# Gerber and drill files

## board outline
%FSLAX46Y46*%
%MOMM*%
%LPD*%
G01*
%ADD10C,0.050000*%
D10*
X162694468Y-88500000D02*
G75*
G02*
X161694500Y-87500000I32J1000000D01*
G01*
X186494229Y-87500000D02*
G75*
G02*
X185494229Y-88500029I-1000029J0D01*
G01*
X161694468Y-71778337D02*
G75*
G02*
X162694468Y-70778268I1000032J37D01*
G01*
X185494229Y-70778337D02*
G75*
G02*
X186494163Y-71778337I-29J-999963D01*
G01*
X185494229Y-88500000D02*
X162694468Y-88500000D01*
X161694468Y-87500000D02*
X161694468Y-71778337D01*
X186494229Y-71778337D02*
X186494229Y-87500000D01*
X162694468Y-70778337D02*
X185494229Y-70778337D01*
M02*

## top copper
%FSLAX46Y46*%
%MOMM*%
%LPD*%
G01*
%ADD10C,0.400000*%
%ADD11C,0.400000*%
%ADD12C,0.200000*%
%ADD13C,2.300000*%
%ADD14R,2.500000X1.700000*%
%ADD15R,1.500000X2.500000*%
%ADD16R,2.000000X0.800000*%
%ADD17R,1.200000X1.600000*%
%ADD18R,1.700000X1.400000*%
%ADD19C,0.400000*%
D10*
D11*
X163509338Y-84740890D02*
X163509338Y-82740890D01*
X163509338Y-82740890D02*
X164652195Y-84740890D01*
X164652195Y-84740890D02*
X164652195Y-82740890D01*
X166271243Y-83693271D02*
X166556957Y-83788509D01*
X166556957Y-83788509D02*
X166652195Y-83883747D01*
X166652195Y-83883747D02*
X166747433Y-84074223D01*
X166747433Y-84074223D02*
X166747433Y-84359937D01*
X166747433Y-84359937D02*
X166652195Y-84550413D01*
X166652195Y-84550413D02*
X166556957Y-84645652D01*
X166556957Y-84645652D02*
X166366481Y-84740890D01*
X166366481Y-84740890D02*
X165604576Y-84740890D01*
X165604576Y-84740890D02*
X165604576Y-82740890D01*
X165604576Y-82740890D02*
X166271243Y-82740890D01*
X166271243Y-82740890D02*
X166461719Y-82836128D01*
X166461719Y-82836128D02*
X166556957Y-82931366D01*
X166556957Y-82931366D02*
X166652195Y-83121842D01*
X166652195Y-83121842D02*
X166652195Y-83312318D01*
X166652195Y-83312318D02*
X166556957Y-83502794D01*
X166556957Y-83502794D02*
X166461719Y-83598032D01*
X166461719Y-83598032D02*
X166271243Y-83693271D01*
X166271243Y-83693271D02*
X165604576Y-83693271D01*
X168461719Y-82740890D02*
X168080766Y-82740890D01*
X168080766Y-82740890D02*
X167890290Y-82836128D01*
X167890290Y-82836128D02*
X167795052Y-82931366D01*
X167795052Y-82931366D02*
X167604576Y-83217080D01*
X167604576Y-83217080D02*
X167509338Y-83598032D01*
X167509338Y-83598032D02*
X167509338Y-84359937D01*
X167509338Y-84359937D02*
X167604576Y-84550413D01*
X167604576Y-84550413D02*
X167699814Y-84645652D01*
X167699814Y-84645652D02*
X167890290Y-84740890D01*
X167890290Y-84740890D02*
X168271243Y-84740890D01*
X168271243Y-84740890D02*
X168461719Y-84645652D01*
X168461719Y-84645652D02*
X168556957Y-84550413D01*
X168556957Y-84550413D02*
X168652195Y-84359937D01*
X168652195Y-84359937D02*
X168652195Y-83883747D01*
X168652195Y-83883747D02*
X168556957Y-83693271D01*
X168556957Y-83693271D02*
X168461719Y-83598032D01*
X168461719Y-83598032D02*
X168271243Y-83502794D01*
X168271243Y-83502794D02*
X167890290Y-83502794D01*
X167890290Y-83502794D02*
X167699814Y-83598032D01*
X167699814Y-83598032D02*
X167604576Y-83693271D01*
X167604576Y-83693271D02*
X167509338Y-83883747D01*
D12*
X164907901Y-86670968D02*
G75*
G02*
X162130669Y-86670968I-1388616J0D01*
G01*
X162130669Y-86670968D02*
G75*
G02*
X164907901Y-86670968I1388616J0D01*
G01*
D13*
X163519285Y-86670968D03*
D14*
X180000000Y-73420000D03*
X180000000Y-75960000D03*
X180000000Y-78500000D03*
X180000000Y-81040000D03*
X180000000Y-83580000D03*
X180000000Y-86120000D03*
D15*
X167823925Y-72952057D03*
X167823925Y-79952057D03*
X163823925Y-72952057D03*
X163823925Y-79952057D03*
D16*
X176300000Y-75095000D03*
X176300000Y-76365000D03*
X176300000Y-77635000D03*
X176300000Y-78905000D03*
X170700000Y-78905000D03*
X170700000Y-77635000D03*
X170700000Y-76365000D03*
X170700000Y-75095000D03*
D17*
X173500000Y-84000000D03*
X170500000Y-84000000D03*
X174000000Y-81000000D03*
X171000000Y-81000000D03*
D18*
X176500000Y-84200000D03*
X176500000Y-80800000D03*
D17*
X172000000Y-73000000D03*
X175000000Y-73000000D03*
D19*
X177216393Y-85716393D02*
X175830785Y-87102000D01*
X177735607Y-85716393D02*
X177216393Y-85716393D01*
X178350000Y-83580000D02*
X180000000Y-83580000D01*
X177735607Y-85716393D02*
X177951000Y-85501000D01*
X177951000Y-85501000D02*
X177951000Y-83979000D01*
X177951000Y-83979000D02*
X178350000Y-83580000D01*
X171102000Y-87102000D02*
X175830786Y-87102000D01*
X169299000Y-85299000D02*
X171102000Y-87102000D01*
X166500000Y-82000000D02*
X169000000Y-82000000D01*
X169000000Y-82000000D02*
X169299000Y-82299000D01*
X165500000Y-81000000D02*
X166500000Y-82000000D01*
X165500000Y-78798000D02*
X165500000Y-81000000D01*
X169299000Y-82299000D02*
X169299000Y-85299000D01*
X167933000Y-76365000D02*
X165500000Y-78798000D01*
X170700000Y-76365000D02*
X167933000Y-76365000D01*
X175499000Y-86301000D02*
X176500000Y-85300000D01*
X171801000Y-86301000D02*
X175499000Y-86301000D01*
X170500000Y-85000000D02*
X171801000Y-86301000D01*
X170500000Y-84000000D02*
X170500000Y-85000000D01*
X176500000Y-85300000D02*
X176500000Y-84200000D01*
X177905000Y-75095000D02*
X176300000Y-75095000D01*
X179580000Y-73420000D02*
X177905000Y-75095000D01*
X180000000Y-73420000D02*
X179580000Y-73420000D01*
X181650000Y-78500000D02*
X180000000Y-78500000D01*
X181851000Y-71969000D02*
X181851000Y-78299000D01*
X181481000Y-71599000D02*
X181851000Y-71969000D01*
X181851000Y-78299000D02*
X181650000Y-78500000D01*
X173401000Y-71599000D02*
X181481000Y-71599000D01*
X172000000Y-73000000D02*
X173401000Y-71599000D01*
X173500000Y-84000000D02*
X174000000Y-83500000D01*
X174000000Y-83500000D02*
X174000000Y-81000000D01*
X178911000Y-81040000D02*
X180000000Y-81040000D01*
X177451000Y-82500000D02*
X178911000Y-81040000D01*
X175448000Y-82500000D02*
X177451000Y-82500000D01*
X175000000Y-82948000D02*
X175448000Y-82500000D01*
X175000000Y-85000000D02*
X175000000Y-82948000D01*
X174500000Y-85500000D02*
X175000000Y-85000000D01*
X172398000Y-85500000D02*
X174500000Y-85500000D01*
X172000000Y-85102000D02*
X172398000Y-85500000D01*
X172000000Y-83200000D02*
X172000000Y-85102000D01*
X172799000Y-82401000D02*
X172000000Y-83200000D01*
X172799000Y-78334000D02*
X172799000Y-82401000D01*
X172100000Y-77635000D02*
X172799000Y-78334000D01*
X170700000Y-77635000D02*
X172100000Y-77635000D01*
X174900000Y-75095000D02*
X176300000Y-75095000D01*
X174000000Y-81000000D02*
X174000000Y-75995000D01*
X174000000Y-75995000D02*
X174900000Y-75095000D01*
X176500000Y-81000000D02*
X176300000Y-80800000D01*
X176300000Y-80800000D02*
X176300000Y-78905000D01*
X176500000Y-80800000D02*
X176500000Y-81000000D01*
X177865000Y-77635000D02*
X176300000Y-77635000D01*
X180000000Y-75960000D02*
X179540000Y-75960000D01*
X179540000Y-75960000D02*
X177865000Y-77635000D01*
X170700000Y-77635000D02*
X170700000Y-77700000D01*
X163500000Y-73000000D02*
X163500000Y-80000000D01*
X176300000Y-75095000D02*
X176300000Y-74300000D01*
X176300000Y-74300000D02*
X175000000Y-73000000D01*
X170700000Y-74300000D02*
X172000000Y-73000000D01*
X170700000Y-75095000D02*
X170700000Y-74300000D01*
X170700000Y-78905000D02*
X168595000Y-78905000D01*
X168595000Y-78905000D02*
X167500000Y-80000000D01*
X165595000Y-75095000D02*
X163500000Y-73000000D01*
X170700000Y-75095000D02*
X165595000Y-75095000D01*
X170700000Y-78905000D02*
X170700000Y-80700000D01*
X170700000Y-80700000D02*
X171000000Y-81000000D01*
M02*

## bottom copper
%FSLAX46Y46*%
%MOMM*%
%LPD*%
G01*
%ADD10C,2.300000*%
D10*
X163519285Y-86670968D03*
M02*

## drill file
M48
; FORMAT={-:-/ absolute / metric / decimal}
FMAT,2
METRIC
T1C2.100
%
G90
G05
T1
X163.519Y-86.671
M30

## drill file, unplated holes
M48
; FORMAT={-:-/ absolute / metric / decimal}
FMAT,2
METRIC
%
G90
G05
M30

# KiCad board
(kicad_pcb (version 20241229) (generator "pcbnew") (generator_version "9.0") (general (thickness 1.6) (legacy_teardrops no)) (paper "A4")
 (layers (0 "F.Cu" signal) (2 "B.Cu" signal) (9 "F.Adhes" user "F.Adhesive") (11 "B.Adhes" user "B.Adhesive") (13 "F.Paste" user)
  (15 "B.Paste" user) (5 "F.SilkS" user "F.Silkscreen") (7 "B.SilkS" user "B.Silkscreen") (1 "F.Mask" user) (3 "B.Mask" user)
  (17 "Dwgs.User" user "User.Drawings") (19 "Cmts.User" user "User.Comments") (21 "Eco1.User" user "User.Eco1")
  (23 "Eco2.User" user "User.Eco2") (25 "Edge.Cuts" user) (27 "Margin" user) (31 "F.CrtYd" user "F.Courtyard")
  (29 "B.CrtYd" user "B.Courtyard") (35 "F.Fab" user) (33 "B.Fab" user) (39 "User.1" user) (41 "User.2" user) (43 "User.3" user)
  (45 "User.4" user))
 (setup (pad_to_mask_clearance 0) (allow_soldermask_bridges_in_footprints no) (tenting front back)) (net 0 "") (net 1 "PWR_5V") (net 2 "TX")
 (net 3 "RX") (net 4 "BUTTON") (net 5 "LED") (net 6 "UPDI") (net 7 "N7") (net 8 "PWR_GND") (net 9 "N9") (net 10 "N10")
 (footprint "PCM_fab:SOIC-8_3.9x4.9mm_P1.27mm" (layer "F.Cu") (at 173.5 77)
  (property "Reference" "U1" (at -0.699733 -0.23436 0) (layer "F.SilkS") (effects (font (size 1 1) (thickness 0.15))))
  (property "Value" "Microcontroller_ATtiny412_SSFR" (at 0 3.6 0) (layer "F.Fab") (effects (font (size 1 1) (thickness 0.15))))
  (pad "1" smd rect (at -2.8 -1.905) (size 2 0.8) (layers "F.Cu" "F.Mask" "F.Paste") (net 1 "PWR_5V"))
  (pad "2" smd rect (at -2.8 -0.635) (size 2 0.8) (layers "F.Cu" "F.Mask" "F.Paste") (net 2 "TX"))
  (pad "3" smd rect (at -2.8 0.635) (size 2 0.8) (layers "F.Cu" "F.Mask" "F.Paste") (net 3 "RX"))
  (pad "4" smd rect (at -2.8 1.905) (size 2 0.8) (layers "F.Cu" "F.Mask" "F.Paste") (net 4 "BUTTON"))
  (pad "5" smd rect (at 2.8 1.905) (size 2 0.8) (layers "F.Cu" "F.Mask" "F.Paste") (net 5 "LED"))
  (pad "6" smd rect (at 2.8 0.635) (size 2 0.8) (layers "F.Cu" "F.Mask" "F.Paste") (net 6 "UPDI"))
  (pad "7" smd rect (at 2.8 -0.635) (size 2 0.8) (layers "F.Cu" "F.Mask" "F.Paste") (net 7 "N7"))
  (pad "8" smd rect (at 2.8 -1.905) (size 2 0.8) (layers "F.Cu" "F.Mask" "F.Paste") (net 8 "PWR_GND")))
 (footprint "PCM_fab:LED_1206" (layer "F.Cu") (at 176.5 82.5 90)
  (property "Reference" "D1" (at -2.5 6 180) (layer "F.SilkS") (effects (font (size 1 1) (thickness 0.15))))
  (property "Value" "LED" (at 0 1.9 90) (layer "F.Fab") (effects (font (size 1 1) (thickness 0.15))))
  (pad "1" smd rect (at -1.7 0 90) (size 1.4 1.7) (layers "F.Cu" "F.Mask" "F.Paste") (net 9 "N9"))
  (pad "2" smd rect (at 1.7 0 90) (size 1.4 1.7) (layers "F.Cu" "F.Mask" "F.Paste") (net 5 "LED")))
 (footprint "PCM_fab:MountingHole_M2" (layer "F.Cu") (at 163.519285 86.670968)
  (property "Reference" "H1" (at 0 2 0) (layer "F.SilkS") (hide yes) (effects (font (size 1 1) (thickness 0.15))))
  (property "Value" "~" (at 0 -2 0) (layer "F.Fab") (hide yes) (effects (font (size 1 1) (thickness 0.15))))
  (pad "" thru_hole circle (at 0 0) (size 2.3 2.3) (drill 2.1) (layers "*.Cu" "*.Mask") (remove_unused_layers no)))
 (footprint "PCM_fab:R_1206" (layer "F.Cu") (at 172 84 180)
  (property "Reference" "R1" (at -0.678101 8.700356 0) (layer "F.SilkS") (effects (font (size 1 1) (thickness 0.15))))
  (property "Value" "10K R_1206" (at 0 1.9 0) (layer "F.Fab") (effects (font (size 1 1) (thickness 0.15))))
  (pad "1" smd rect (at -1.5 0 180) (size 1.2 1.6) (layers "F.Cu" "F.Mask" "F.Paste") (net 8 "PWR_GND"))
  (pad "2" smd rect (at 1.5 0 180) (size 1.2 1.6) (layers "F.Cu" "F.Mask" "F.Paste") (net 9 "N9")))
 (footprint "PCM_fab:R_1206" (layer "F.Cu") (at 172.5 81 180)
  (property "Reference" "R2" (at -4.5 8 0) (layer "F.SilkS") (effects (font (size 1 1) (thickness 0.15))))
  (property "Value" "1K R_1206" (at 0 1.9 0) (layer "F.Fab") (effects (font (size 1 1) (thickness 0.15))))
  (pad "1" smd rect (at -1.5 0 180) (size 1.2 1.6) (layers "F.Cu" "F.Mask" "F.Paste") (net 8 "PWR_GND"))
  (pad "2" smd rect (at 1.5 0 180) (size 1.2 1.6) (layers "F.Cu" "F.Mask" "F.Paste") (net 4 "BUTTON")))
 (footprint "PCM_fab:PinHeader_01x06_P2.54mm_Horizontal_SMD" (layer "F.Cu") (at 180 73.42)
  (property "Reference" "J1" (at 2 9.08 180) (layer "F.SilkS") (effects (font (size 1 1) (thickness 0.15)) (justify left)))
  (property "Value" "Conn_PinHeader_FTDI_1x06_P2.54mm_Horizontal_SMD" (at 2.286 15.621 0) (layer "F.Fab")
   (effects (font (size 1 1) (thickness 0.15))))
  (pad "1" smd rect (at 0 0) (size 2.5 1.7) (layers "F.Cu" "F.Mask" "F.Paste") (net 8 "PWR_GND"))
  (pad "2" smd rect (at 0 2.54) (size 2.5 1.7) (layers "F.Cu" "F.Mask" "F.Paste") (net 6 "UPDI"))
  (pad "3" smd rect (at 0 5.08) (size 2.5 1.7) (layers "F.Cu" "F.Mask" "F.Paste") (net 1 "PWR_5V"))
  (pad "4" smd rect (at 0 7.62) (size 2.5 1.7) (layers "F.Cu" "F.Mask" "F.Paste") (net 3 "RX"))
  (pad "5" smd rect (at 0 10.16) (size 2.5 1.7) (layers "F.Cu" "F.Mask" "F.Paste") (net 2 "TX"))
  (pad "6" smd rect (at 0 12.7) (size 2.5 1.7) (layers "F.Cu" "F.Mask" "F.Paste") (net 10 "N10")))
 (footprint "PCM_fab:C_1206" (layer "F.Cu") (at 173.5 73)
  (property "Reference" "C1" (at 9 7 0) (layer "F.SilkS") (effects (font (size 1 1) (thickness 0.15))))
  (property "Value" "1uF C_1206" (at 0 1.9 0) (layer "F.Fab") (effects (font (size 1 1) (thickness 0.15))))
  (pad "1" smd rect (at -1.5 0) (size 1.2 1.6) (layers "F.Cu" "F.Mask" "F.Paste") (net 1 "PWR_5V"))
  (pad "2" smd rect (at 1.5 0) (size 1.2 1.6) (layers "F.Cu" "F.Mask" "F.Paste") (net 8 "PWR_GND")))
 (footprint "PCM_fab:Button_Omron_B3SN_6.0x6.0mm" (layer "F.Cu") (at 165.823925 76.452057 90)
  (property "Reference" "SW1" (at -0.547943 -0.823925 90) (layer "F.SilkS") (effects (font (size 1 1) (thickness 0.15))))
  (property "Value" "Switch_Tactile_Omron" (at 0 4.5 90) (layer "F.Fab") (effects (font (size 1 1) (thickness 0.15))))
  (pad "1" smd rect (at -3.5 -2 90) (size 2.5 1.5) (layers "F.Cu" "F.Mask" "F.Paste") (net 1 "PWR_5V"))
  (pad "1" smd rect (at 3.5 -2 90) (size 2.5 1.5) (layers "F.Cu" "F.Mask" "F.Paste") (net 1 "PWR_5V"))
  (pad "2" smd rect (at -3.5 2 90) (size 2.5 1.5) (layers "F.Cu" "F.Mask" "F.Paste") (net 4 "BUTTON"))
  (pad "2" smd rect (at 3.5 2 90) (size 2.5 1.5) (layers "F.Cu" "F.Mask" "F.Paste") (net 4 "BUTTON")))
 (gr_circle (center 163.519285 86.670968) (end 162.636568 87.742912) (stroke (width 0.2) (type default)) (fill no) (layer "F.Cu"))
 (gr_arc (start 162.694468 88.5) (mid 161.987382 88.207095) (end 161.694468 87.5) (stroke (width 0.05) (type default)) (layer "Edge.Cuts"))
 (gr_line (start 162.694468 70.778337) (end 185.494229 70.778337) (stroke (width 0.05) (type default)) (layer "Edge.Cuts"))
 (gr_line (start 185.494229 88.5) (end 162.694468 88.5) (stroke (width 0.05) (type default)) (layer "Edge.Cuts"))
 (gr_line (start 186.494229 71.778337) (end 186.494229 87.5) (stroke (width 0.05) (type default)) (layer "Edge.Cuts"))
 (gr_arc (start 161.694468 71.778337) (mid 161.987346 71.071195) (end 162.694468 70.778337) (stroke (width 0.05) (type default))
  (layer "Edge.Cuts"))
 (gr_arc (start 185.494229 70.778337) (mid 186.201336 71.07123) (end 186.494229 71.778337) (stroke (width 0.05) (type default))
  (layer "Edge.Cuts"))
 (gr_line (start 161.694468 87.5) (end 161.694468 71.778337) (stroke (width 0.05) (type default)) (layer "Edge.Cuts"))
 (gr_arc (start 186.494229 87.5) (mid 186.201336 88.207107) (end 185.494229 88.5) (stroke (width 0.05) (type default)) (layer "Edge.Cuts"))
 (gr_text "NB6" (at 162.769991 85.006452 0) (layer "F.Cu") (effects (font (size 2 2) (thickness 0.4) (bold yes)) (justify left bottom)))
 (segment (start 165.595 75.095) (end 163.5 73) (width 0.4) (layer "F.Cu") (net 1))
 (segment (start 170.7 75.095) (end 170.7 74.3) (width 0.4) (layer "F.Cu") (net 1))
 (segment (start 170.7 74.3) (end 172 73) (width 0.4) (layer "F.Cu") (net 1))
 (segment (start 170.7 75.095) (end 165.595 75.095) (width 0.4) (layer "F.Cu") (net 1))
 (segment (start 173.401 71.599) (end 181.481 71.599) (width 0.4) (layer "F.Cu") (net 1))
 (segment (start 172 73) (end 173.401 71.599) (width 0.4) (layer "F.Cu") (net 1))
 (segment (start 181.65 78.5) (end 180 78.5) (width 0.4) (layer "F.Cu") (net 1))
 (segment (start 181.851 78.299) (end 181.65 78.5) (width 0.4) (layer "F.Cu") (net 1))
 (segment (start 163.5 73) (end 163.5 80) (width 0.4) (layer "F.Cu") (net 1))
 (segment (start 181.851 71.969) (end 181.851 78.299) (width 0.4) (layer "F.Cu") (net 1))
 (segment (start 181.481 71.599) (end 181.851 71.969) (width 0.4) (layer "F.Cu") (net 1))
 (segment (start 175.499 86.301) (end 176.5 85.3) (width 0.4) (layer "F.Cu") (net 9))
 (segment (start 170.5 84) (end 170.5 85) (width 0.4) (layer "F.Cu") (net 9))
 (segment (start 171.801 86.301) (end 175.499 86.301) (width 0.4) (layer "F.Cu") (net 9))
 (segment (start 170.5 85) (end 171.801 86.301) (width 0.4) (layer "F.Cu") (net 9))
 (segment (start 176.5 85.3) (end 176.5 84.2) (width 0.4) (layer "F.Cu") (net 9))
 (segment (start 174 75.995) (end 174.9 75.095) (width 0.4) (layer "F.Cu") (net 8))
 (segment (start 176.3 75.095) (end 176.3 74.3) (width 0.4) (layer "F.Cu") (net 8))
 (segment (start 174.9 75.095) (end 176.3 75.095) (width 0.4) (layer "F.Cu") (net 8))
 (segment (start 179.58 73.42) (end 177.905 75.095) (width 0.4) (layer "F.Cu") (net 8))
 (segment (start 173.5 84) (end 174 83.5) (width 0.4) (layer "F.Cu") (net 8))
 (segment (start 176.3 74.3) (end 175 73) (width 0.4) (layer "F.Cu") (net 8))
 (segment (start 174 81) (end 174 75.995) (width 0.4) (layer "F.Cu") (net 8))
 (segment (start 174 83.5) (end 174 81) (width 0.4) (layer "F.Cu") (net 8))
 (segment (start 180 73.42) (end 179.58 73.42) (width 0.4) (layer "F.Cu") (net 8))
 (segment (start 177.905 75.095) (end 176.3 75.095) (width 0.4) (layer "F.Cu") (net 8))
 (segment (start 176.5 81) (end 176.3 80.8) (width 0.4) (layer "F.Cu") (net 5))
 (segment (start 176.5 80.8) (end 176.5 81) (width 0.4) (layer "F.Cu") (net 5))
 (segment (start 176.3 80.8) (end 176.3 78.905) (width 0.4) (layer "F.Cu") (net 5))
 (segment (start 169.299 85.299) (end 171.102 87.102) (width 0.4) (layer "F.Cu") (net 2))
 (segment (start 167.933 76.365) (end 165.5 78.798) (width 0.4) (layer "F.Cu") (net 2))
 (segment (start 177.735607 85.716393) (end 177.216393 85.716393) (width 0.4) (layer "F.Cu") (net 2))
 (segment (start 178.35 83.58) (end 180 83.58) (width 0.4) (layer "F.Cu") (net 2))
 (segment (start 171.102 87.102) (end 175.830786 87.102) (width 0.4) (layer "F.Cu") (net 2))
 (segment (start 177.951 85.501) (end 177.951 83.979) (width 0.4) (layer "F.Cu") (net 2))
 (segment (start 170.7 76.365) (end 167.933 76.365) (width 0.4) (layer "F.Cu") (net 2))
 (segment (start 169.299 82.299) (end 169.299 85.299) (width 0.4) (layer "F.Cu") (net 2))
 (segment (start 177.951 83.979) (end 178.35 83.58) (width 0.4) (layer "F.Cu") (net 2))
 (segment (start 169 82) (end 169.299 82.299) (width 0.4) (layer "F.Cu") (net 2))
 (segment (start 165.5 81) (end 166.5 82) (width 0.4) (layer "F.Cu") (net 2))
 (segment (start 177.735607 85.716393) (end 177.951 85.501) (width 0.4) (layer "F.Cu") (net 2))
 (segment (start 177.216393 85.716393) (end 175.830785 87.102) (width 0.4) (layer "F.Cu") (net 2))
 (segment (start 165.5 78.798) (end 165.5 81) (width 0.4) (layer "F.Cu") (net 2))
 (segment (start 166.5 82) (end 169 82) (width 0.4) (layer "F.Cu") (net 2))
 (segment (start 172.398 85.5) (end 174.5 85.5) (width 0.4) (layer "F.Cu") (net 3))
 (segment (start 172 85.102) (end 172.398 85.5) (width 0.4) (layer "F.Cu") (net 3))
 (segment (start 172.799 78.334) (end 172.799 82.401) (width 0.4) (layer "F.Cu") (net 3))
 (segment (start 172 83.2) (end 172 85.102) (width 0.4) (layer "F.Cu") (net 3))
 (segment (start 172.1 77.635) (end 172.799 78.334) (width 0.4) (layer "F.Cu") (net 3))
 (segment (start 172.799 82.401) (end 172 83.2) (width 0.4) (layer "F.Cu") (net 3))
 (segment (start 174.5 85.5) (end 175 85) (width 0.4) (layer "F.Cu") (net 3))
 (segment (start 177.451 82.5) (end 178.911 81.04) (width 0.4) (layer "F.Cu") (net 3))
 (segment (start 175.448 82.5) (end 177.451 82.5) (width 0.4) (layer "F.Cu") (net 3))
 (segment (start 170.7 77.635) (end 170.7 77.7) (width 0.4) (layer "F.Cu") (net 3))
 (segment (start 170.7 77.635) (end 172.1 77.635) (width 0.4) (layer "F.Cu") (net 3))
 (segment (start 175 85) (end 175 82.948) (width 0.4) (layer "F.Cu") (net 3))
 (segment (start 175 82.948) (end 175.448 82.5) (width 0.4) (layer "F.Cu") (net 3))
 (segment (start 178.911 81.04) (end 180 81.04) (width 0.4) (layer "F.Cu") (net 3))
 (segment (start 168.595 78.905) (end 167.5 80) (width 0.4) (layer "F.Cu") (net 4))
 (segment (start 170.7 80.7) (end 171 81) (width 0.4) (layer "F.Cu") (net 4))
 (segment (start 170.7 78.905) (end 168.595 78.905) (width 0.4) (layer "F.Cu") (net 4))
 (segment (start 170.7 78.905) (end 170.7 80.7) (width 0.4) (layer "F.Cu") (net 4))
 (segment (start 177.865 77.635) (end 176.3 77.635) (width 0.4) (layer "F.Cu") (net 6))
 (segment (start 180 75.96) (end 179.54 75.96) (width 0.4) (layer "F.Cu") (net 6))
 (segment (start 179.54 75.96) (end 177.865 77.635) (width 0.4) (layer "F.Cu") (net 6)))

